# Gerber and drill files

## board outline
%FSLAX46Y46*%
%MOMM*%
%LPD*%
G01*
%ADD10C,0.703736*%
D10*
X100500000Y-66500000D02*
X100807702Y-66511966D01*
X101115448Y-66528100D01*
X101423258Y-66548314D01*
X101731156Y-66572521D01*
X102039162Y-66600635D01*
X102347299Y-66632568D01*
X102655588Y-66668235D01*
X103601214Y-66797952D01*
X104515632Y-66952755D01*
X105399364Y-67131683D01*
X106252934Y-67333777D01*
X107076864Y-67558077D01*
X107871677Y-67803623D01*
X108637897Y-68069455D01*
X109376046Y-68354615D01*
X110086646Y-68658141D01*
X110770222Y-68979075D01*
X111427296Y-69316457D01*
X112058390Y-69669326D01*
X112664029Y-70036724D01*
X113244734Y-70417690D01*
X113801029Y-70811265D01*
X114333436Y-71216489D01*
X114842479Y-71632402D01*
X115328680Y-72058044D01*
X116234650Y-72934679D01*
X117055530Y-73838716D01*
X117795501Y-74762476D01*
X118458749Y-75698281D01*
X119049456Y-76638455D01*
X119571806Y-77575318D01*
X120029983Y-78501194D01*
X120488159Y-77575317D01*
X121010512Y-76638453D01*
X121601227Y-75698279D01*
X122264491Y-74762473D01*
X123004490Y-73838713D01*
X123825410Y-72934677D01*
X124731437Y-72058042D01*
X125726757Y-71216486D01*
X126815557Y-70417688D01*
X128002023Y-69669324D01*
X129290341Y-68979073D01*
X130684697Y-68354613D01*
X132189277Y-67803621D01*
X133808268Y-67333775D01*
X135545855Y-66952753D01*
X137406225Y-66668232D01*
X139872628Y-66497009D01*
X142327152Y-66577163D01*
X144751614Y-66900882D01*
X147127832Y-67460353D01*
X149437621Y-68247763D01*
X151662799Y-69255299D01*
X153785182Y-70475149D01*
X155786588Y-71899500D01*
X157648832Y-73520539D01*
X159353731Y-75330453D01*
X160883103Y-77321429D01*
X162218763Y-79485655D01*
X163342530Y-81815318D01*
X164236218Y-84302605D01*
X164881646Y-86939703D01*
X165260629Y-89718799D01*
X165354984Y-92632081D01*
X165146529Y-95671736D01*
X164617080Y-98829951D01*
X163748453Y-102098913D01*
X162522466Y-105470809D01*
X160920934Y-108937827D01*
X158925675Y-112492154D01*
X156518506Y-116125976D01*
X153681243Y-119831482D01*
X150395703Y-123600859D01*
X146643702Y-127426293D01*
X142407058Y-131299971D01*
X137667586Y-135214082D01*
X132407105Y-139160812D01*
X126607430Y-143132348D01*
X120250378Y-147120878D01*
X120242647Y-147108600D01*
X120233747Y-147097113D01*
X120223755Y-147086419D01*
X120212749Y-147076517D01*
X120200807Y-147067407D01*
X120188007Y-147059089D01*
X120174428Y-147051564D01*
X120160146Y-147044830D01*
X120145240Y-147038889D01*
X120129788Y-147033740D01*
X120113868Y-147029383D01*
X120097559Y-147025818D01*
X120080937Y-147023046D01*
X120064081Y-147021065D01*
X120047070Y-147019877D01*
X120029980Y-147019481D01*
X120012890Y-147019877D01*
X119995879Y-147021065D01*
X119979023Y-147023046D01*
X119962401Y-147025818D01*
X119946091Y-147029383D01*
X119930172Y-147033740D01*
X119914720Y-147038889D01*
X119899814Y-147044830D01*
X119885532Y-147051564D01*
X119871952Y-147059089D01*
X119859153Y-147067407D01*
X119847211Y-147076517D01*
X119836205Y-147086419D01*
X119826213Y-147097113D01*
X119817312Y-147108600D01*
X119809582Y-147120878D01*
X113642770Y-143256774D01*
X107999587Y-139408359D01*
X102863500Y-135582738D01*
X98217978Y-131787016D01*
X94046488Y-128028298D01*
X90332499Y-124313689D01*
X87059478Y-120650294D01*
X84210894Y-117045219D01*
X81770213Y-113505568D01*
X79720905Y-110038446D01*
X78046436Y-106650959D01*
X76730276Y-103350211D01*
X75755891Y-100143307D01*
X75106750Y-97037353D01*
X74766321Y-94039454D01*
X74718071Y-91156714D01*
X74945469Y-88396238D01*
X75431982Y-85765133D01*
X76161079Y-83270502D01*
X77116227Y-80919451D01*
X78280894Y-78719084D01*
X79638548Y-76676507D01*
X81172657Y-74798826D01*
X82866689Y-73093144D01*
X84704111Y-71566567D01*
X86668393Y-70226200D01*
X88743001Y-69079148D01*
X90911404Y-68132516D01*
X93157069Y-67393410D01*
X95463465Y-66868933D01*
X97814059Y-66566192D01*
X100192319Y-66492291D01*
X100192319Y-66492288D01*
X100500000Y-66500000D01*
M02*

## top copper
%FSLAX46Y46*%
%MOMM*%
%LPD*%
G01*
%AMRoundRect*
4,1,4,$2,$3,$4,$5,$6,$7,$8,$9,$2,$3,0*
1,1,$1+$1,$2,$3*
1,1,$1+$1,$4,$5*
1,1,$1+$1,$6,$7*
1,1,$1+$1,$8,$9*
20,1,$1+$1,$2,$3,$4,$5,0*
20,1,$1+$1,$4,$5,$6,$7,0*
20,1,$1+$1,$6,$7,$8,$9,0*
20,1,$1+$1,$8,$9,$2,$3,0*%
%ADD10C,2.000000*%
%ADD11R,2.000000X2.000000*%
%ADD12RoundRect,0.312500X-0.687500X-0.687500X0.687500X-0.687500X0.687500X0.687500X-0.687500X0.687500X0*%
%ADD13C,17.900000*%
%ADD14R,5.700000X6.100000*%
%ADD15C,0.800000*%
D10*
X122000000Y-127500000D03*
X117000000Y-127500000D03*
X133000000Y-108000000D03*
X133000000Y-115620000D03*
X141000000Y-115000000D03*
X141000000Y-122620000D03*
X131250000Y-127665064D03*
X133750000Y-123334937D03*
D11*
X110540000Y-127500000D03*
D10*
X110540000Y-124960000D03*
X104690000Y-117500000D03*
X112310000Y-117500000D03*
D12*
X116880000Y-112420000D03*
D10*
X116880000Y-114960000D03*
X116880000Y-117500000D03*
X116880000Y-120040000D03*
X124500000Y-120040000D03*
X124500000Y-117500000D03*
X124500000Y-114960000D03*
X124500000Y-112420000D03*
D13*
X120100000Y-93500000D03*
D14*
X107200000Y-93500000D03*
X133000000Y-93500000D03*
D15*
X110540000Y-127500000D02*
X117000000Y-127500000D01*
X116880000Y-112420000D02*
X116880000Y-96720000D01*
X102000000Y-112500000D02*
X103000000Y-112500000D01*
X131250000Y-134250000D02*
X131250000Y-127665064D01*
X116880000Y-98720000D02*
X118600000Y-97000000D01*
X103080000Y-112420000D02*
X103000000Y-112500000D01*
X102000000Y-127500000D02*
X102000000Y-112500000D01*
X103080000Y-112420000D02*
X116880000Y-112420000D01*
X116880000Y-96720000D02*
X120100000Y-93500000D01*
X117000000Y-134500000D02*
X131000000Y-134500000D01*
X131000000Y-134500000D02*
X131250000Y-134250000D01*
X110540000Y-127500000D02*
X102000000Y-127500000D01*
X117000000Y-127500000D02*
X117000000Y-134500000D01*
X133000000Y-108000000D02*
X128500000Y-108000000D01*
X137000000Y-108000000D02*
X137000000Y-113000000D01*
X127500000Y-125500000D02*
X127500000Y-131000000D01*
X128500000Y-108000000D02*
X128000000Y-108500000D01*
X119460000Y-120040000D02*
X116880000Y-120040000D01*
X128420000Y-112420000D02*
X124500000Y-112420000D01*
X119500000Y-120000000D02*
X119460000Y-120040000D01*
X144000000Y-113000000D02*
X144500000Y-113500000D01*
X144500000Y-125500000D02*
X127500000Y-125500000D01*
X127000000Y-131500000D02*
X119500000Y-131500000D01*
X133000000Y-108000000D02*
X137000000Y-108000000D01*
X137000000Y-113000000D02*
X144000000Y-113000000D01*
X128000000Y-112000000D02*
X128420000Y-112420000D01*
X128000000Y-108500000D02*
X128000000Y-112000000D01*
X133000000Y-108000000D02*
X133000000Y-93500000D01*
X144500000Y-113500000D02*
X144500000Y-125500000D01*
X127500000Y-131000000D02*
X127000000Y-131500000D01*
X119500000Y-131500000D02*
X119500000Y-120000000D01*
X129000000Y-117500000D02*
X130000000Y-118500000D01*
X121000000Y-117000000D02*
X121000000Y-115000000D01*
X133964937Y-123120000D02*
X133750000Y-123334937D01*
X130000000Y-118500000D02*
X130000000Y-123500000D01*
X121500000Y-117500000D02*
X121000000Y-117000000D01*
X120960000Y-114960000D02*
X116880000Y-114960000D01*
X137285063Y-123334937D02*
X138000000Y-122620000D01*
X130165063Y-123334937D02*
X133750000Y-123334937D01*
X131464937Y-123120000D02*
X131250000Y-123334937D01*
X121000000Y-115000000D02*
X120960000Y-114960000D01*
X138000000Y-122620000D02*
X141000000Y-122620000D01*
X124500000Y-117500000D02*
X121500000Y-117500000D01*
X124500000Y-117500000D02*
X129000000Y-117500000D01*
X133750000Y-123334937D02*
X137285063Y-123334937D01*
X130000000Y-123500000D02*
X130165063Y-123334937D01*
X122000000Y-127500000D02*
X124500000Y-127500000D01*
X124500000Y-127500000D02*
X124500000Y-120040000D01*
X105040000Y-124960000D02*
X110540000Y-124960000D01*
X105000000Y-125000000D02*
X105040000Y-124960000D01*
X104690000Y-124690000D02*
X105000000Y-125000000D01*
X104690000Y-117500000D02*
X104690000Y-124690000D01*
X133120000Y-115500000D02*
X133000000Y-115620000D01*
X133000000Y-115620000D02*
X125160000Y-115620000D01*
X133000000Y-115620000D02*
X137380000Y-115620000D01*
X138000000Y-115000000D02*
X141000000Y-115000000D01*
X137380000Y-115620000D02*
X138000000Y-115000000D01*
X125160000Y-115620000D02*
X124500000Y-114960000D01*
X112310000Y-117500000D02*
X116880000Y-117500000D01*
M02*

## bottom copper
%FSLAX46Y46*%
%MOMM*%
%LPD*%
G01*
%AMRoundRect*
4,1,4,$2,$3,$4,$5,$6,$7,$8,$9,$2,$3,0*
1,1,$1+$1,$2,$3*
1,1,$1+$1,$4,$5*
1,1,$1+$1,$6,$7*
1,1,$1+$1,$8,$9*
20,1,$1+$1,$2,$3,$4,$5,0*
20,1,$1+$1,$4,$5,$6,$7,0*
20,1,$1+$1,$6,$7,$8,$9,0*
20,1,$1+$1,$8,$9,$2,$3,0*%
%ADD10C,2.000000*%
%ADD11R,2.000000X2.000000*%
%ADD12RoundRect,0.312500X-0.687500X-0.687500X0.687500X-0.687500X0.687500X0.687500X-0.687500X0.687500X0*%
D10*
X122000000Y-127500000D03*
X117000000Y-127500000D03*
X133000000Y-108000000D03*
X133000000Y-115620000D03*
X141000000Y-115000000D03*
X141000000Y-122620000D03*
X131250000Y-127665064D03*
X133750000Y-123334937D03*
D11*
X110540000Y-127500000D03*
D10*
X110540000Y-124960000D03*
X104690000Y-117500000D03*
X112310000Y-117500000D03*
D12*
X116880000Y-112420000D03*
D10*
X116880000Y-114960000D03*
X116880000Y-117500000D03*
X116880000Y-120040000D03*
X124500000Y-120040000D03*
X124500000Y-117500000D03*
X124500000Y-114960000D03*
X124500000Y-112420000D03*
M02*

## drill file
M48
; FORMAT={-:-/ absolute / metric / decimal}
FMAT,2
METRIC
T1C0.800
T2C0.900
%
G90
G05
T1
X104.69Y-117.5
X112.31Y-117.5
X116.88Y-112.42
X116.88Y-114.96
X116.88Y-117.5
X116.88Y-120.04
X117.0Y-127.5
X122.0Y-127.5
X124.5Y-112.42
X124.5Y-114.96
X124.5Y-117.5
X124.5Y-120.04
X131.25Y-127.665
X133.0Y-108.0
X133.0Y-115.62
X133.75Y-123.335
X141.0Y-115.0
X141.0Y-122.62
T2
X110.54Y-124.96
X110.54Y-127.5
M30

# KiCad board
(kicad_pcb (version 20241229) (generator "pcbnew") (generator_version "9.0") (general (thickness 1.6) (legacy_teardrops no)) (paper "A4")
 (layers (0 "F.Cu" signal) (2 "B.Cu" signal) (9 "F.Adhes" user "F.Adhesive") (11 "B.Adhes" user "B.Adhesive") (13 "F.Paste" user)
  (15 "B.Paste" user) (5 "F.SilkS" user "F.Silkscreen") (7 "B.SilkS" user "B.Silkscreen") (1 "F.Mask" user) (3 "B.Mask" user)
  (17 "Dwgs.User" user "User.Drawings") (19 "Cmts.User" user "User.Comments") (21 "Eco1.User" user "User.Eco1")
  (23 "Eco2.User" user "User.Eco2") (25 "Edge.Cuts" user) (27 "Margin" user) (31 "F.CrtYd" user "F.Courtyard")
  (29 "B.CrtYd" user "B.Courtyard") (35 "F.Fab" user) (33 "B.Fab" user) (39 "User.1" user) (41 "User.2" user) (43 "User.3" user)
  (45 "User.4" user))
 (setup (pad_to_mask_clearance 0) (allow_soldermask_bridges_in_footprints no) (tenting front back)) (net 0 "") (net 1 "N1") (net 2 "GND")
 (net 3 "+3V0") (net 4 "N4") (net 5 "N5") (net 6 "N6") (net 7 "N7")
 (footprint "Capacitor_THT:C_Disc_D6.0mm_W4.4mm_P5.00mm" (layer "F.Cu") (at 122 127.5 180)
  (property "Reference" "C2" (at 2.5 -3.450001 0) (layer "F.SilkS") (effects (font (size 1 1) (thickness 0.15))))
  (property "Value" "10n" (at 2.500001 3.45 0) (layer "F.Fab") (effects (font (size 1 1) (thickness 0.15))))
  (pad "1" thru_hole circle (at 0 0 180) (size 2 2) (drill 0.8) (layers "*.Cu" "*.Mask") (remove_unused_layers no) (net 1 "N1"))
  (pad "2" thru_hole circle (at 5 0 180) (size 2 2) (drill 0.8) (layers "*.Cu" "*.Mask") (remove_unused_layers no) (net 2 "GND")))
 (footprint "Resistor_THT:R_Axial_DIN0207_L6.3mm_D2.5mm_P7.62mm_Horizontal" (layer "F.Cu") (at 133 108 -90)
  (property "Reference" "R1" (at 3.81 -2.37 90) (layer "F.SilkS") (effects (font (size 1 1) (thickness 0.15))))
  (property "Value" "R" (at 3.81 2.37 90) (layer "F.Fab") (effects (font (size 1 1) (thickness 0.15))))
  (pad "1" thru_hole circle (at 0 0 270) (size 2 2) (drill 0.8) (layers "*.Cu" "*.Mask") (remove_unused_layers no) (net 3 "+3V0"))
  (pad "2" thru_hole circle (at 7.62 0 270) (size 2 2) (drill 0.8) (layers "*.Cu" "*.Mask") (remove_unused_layers no) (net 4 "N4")))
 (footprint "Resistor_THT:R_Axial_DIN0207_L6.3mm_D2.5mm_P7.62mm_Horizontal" (layer "F.Cu") (at 141 115 -90)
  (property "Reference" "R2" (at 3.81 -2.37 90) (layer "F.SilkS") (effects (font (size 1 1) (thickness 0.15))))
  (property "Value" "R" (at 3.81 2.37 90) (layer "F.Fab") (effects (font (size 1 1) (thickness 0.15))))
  (pad "1" thru_hole circle (at 0 0 270) (size 2 2) (drill 0.8) (layers "*.Cu" "*.Mask") (remove_unused_layers no) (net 4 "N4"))
  (pad "2" thru_hole circle (at 7.62 0 270) (size 2 2) (drill 0.8) (layers "*.Cu" "*.Mask") (remove_unused_layers no) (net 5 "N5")))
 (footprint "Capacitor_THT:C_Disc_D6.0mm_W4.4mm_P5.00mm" (layer "F.Cu") (at 131.25 127.665064 60)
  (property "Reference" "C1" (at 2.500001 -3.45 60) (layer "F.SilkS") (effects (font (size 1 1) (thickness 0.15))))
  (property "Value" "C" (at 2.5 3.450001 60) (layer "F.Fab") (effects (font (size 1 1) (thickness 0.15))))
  (pad "1" thru_hole circle (at 0 0 60) (size 2 2) (drill 0.8) (layers "*.Cu" "*.Mask") (remove_unused_layers no) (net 2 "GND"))
  (pad "2" thru_hole circle (at 5 0 60) (size 2 2) (drill 0.8) (layers "*.Cu" "*.Mask") (remove_unused_layers no) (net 5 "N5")))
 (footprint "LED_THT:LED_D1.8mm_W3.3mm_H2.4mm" (layer "F.Cu") (at 110.54 127.5 90)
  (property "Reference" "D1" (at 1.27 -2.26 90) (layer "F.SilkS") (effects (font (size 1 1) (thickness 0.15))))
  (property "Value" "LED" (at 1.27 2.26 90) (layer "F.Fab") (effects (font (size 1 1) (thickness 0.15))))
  (pad "1" thru_hole rect (at 0 0 90) (size 2 2) (drill 0.9) (layers "*.Cu" "*.Mask") (remove_unused_layers no) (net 2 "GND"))
  (pad "2" thru_hole circle (at 2.54 0 90) (size 2 2) (drill 0.9) (layers "*.Cu" "*.Mask") (remove_unused_layers no) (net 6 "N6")))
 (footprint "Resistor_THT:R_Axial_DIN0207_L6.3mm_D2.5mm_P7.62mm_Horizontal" (layer "F.Cu") (at 104.69 117.5)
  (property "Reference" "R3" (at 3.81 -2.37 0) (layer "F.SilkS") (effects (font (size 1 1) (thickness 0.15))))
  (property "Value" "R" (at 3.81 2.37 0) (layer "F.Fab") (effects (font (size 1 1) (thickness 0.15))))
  (pad "1" thru_hole circle (at 0 0) (size 2 2) (drill 0.8) (layers "*.Cu" "*.Mask") (remove_unused_layers no) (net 6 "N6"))
  (pad "2" thru_hole circle (at 7.62 0) (size 2 2) (drill 0.8) (layers "*.Cu" "*.Mask") (remove_unused_layers no) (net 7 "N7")))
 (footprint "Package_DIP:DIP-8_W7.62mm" (layer "F.Cu") (at 116.88 112.42)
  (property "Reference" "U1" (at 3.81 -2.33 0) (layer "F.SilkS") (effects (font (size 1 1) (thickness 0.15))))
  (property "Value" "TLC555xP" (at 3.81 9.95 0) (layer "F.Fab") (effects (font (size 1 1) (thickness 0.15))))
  (pad "1" thru_hole roundrect (at 0 0) (size 2 2) (drill 0.8) (layers "*.Cu" "*.Mask") (remove_unused_layers no) (roundrect_rratio 0.15625)
   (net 2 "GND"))
  (pad "2" thru_hole circle (at 0 2.54) (size 2 2) (drill 0.8) (layers "*.Cu" "*.Mask") (remove_unused_layers no) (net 5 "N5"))
  (pad "3" thru_hole circle (at 0 5.08) (size 2 2) (drill 0.8) (layers "*.Cu" "*.Mask") (remove_unused_layers no) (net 7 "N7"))
  (pad "4" thru_hole circle (at 0 7.62) (size 2 2) (drill 0.8) (layers "*.Cu" "*.Mask") (remove_unused_layers no) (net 3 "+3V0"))
  (pad "5" thru_hole circle (at 7.62 7.62) (size 2 2) (drill 0.8) (layers "*.Cu" "*.Mask") (remove_unused_layers no) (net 1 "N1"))
  (pad "6" thru_hole circle (at 7.62 5.08) (size 2 2) (drill 0.8) (layers "*.Cu" "*.Mask") (remove_unused_layers no) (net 5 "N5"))
  (pad "7" thru_hole circle (at 7.62 2.54) (size 2 2) (drill 0.8) (layers "*.Cu" "*.Mask") (remove_unused_layers no) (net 4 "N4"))
  (pad "8" thru_hole circle (at 7.62 0) (size 2 2) (drill 0.8) (layers "*.Cu" "*.Mask") (remove_unused_layers no) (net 3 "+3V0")))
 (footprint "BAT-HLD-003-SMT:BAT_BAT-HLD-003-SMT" (layer "F.Cu") (at 120.1 93.5)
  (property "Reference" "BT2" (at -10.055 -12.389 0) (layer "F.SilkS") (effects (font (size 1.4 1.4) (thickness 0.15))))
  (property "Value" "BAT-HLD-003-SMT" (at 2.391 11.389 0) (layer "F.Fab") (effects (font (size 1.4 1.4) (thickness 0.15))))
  (pad "N" smd circle (at 0 0) (size 17.9 17.9) (layers "F.Cu" "F.Mask") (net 2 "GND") (solder_mask_margin 0.102))
  (pad "P1" smd rect (at -12.9 0) (size 5.7 6.1) (layers "F.Cu" "F.Mask" "F.Paste") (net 3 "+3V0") (solder_mask_margin 0.102))
  (pad "P2" smd rect (at 12.9 0) (size 5.7 6.1) (layers "F.Cu" "F.Mask" "F.Paste") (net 3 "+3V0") (solder_mask_margin 0.102)))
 (gr_poly
  (pts (xy 100.5 66.5) (xy 100.807702 66.511966) (xy 101.115448 66.5281) (xy 101.423258 66.548314) (xy 101.731156 66.572521)
   (xy 102.039162 66.600635) (xy 102.347299 66.632568) (xy 102.655588 66.668235) (xy 103.601214 66.797952) (xy 104.515632 66.952755)
   (xy 105.399364 67.131683) (xy 106.252934 67.333777) (xy 107.076864 67.558077) (xy 107.871677 67.803623) (xy 108.637897 68.069455)
   (xy 109.376046 68.354615) (xy 110.086646 68.658141) (xy 110.770222 68.979075) (xy 111.427296 69.316457) (xy 112.05839 69.669326)
   (xy 112.664029 70.036724) (xy 113.244734 70.41769) (xy 113.801029 70.811265) (xy 114.333436 71.216489) (xy 114.842479 71.632402)
   (xy 115.32868 72.058044) (xy 116.23465 72.934679) (xy 117.05553 73.838716) (xy 117.795501 74.762476) (xy 118.458749 75.698281)
   (xy 119.049456 76.638455) (xy 119.571806 77.575318) (xy 120.029983 78.501194) (xy 120.488159 77.575317) (xy 121.010512 76.638453)
   (xy 121.601227 75.698279) (xy 122.264491 74.762473) (xy 123.00449 73.838713) (xy 123.82541 72.934677) (xy 124.731437 72.058042)
   (xy 125.726757 71.216486) (xy 126.815557 70.417688) (xy 128.002023 69.669324) (xy 129.290341 68.979073) (xy 130.684697 68.354613)
   (xy 132.189277 67.803621) (xy 133.808268 67.333775) (xy 135.545855 66.952753) (xy 137.406225 66.668232) (xy 139.872628 66.497009)
   (xy 142.327152 66.577163) (xy 144.751614 66.900882) (xy 147.127832 67.460353) (xy 149.437621 68.247763) (xy 151.662799 69.255299)
   (xy 153.785182 70.475149) (xy 155.786588 71.8995) (xy 157.648832 73.520539) (xy 159.353731 75.330453) (xy 160.883103 77.321429)
   (xy 162.218763 79.485655) (xy 163.34253 81.815318) (xy 164.236218 84.302605) (xy 164.881646 86.939703) (xy 165.260629 89.718799)
   (xy 165.354984 92.632081) (xy 165.146529 95.671736) (xy 164.61708 98.829951) (xy 163.748453 102.098913) (xy 162.522466 105.470809)
   (xy 160.920934 108.937827) (xy 158.925675 112.492154) (xy 156.518506 116.125976) (xy 153.681243 119.831482) (xy 150.395703 123.600859)
   (xy 146.643702 127.426293) (xy 142.407058 131.299971) (xy 137.667586 135.214082) (xy 132.407105 139.160812) (xy 126.60743 143.132348)
   (xy 120.250378 147.120878) (xy 120.242647 147.1086) (xy 120.233747 147.097113) (xy 120.223755 147.086419) (xy 120.212749 147.076517)
   (xy 120.200807 147.067407) (xy 120.188007 147.059089) (xy 120.174428 147.051564) (xy 120.160146 147.04483) (xy 120.14524 147.038889)
   (xy 120.129788 147.03374) (xy 120.113868 147.029383) (xy 120.097559 147.025818) (xy 120.080937 147.023046) (xy 120.064081 147.021065)
   (xy 120.04707 147.019877) (xy 120.02998 147.019481) (xy 120.01289 147.019877) (xy 119.995879 147.021065) (xy 119.979023 147.023046)
   (xy 119.962401 147.025818) (xy 119.946091 147.029383) (xy 119.930172 147.03374) (xy 119.91472 147.038889) (xy 119.899814 147.04483)
   (xy 119.885532 147.051564) (xy 119.871952 147.059089) (xy 119.859153 147.067407) (xy 119.847211 147.076517) (xy 119.836205 147.086419)
   (xy 119.826213 147.097113) (xy 119.817312 147.1086) (xy 119.809582 147.120878) (xy 113.64277 143.256774) (xy 107.999587 139.408359)
   (xy 102.8635 135.582738) (xy 98.217978 131.787016) (xy 94.046488 128.028298) (xy 90.332499 124.313689) (xy 87.059478 120.650294)
   (xy 84.210894 117.045219) (xy 81.770213 113.505568) (xy 79.720905 110.038446) (xy 78.046436 106.650959) (xy 76.730276 103.350211)
   (xy 75.755891 100.143307) (xy 75.10675 97.037353) (xy 74.766321 94.039454) (xy 74.718071 91.156714) (xy 74.945469 88.396238)
   (xy 75.431982 85.765133) (xy 76.161079 83.270502) (xy 77.116227 80.919451) (xy 78.280894 78.719084) (xy 79.638548 76.676507)
   (xy 81.172657 74.798826) (xy 82.866689 73.093144) (xy 84.704111 71.566567) (xy 86.668393 70.2262) (xy 88.743001 69.079148)
   (xy 90.911404 68.132516) (xy 93.157069 67.39341) (xy 95.463465 66.868933) (xy 97.814059 66.566192) (xy 100.192319 66.492291)
   (xy 100.192319 66.492288))
  (stroke (width 0.703736) (type solid)) (fill no) (layer "Edge.Cuts"))
 (segment (start 110.54 127.5) (end 117 127.5) (width 0.8) (layer "F.Cu") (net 2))
 (segment (start 116.88 112.42) (end 116.88 96.72) (width 0.8) (layer "F.Cu") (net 2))
 (segment (start 102 112.5) (end 103 112.5) (width 0.8) (layer "F.Cu") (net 2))
 (segment (start 131.25 134.25) (end 131.25 127.665064) (width 0.8) (layer "F.Cu") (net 2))
 (segment (start 116.88 98.72) (end 118.6 97) (width 0.8) (layer "F.Cu") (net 2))
 (segment (start 103.08 112.42) (end 103 112.5) (width 0.8) (layer "F.Cu") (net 2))
 (segment (start 102 127.5) (end 102 112.5) (width 0.8) (layer "F.Cu") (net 2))
 (segment (start 103.08 112.42) (end 116.88 112.42) (width 0.8) (layer "F.Cu") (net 2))
 (segment (start 116.88 96.72) (end 120.1 93.5) (width 0.8) (layer "F.Cu") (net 2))
 (segment (start 117 134.5) (end 131 134.5) (width 0.8) (layer "F.Cu") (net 2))
 (segment (start 131 134.5) (end 131.25 134.25) (width 0.8) (layer "F.Cu") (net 2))
 (segment (start 110.54 127.5) (end 102 127.5) (width 0.8) (layer "F.Cu") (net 2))
 (segment (start 117 127.5) (end 117 134.5) (width 0.8) (layer "F.Cu") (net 2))
 (segment (start 133 108) (end 128.5 108) (width 0.8) (layer "F.Cu") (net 3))
 (segment (start 137 108) (end 137 113) (width 0.8) (layer "F.Cu") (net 3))
 (segment (start 127.5 125.5) (end 127.5 131) (width 0.8) (layer "F.Cu") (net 3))
 (segment (start 128.5 108) (end 128 108.5) (width 0.8) (layer "F.Cu") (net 3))
 (segment (start 119.46 120.04) (end 116.88 120.04) (width 0.8) (layer "F.Cu") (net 3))
 (segment (start 128.42 112.42) (end 124.5 112.42) (width 0.8) (layer "F.Cu") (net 3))
 (segment (start 119.5 120) (end 119.46 120.04) (width 0.8) (layer "F.Cu") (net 3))
 (segment (start 144 113) (end 144.5 113.5) (width 0.8) (layer "F.Cu") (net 3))
 (segment (start 144.5 125.5) (end 127.5 125.5) (width 0.8) (layer "F.Cu") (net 3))
 (segment (start 127 131.5) (end 119.5 131.5) (width 0.8) (layer "F.Cu") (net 3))
 (segment (start 133 108) (end 137 108) (width 0.8) (layer "F.Cu") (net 3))
 (segment (start 137 113) (end 144 113) (width 0.8) (layer "F.Cu") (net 3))
 (segment (start 128 112) (end 128.42 112.42) (width 0.8) (layer "F.Cu") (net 3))
 (segment (start 128 108.5) (end 128 112) (width 0.8) (layer "F.Cu") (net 3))
 (segment (start 133 108) (end 133 93.5) (width 0.8) (layer "F.Cu") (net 3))
 (segment (start 144.5 113.5) (end 144.5 125.5) (width 0.8) (layer "F.Cu") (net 3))
 (segment (start 127.5 131) (end 127 131.5) (width 0.8) (layer "F.Cu") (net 3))
 (segment (start 119.5 131.5) (end 119.5 120) (width 0.8) (layer "F.Cu") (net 3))
 (segment (start 129 117.5) (end 130 118.5) (width 0.8) (layer "F.Cu") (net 5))
 (segment (start 121 117) (end 121 115) (width 0.8) (layer "F.Cu") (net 5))
 (segment (start 133.964937 123.12) (end 133.75 123.334937) (width 0.8) (layer "F.Cu") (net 5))
 (segment (start 130 118.5) (end 130 123.5) (width 0.8) (layer "F.Cu") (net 5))
 (segment (start 121.5 117.5) (end 121 117) (width 0.8) (layer "F.Cu") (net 5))
 (segment (start 120.96 114.96) (end 116.88 114.96) (width 0.8) (layer "F.Cu") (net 5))
 (segment (start 137.285063 123.334937) (end 138 122.62) (width 0.8) (layer "F.Cu") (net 5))
 (segment (start 130.165063 123.334937) (end 133.75 123.334937) (width 0.8) (layer "F.Cu") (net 5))
 (segment (start 131.464937 123.12) (end 131.25 123.334937) (width 0.8) (layer "F.Cu") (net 5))
 (segment (start 121 115) (end 120.96 114.96) (width 0.8) (layer "F.Cu") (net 5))
 (segment (start 138 122.62) (end 141 122.62) (width 0.8) (layer "F.Cu") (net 5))
 (segment (start 124.5 117.5) (end 121.5 117.5) (width 0.8) (layer "F.Cu") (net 5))
 (segment (start 124.5 117.5) (end 129 117.5) (width 0.8) (layer "F.Cu") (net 5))
 (segment (start 133.75 123.334937) (end 137.285063 123.334937) (width 0.8) (layer "F.Cu") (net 5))
 (segment (start 130 123.5) (end 130.165063 123.334937) (width 0.8) (layer "F.Cu") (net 5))
 (segment (start 122 127.5) (end 124.5 127.5) (width 0.8) (layer "F.Cu") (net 1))
 (segment (start 124.5 127.5) (end 124.5 120.04) (width 0.8) (layer "F.Cu") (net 1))
 (segment (start 105.04 124.96) (end 110.54 124.96) (width 0.8) (layer "F.Cu") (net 6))
 (segment (start 105 125) (end 105.04 124.96) (width 0.8) (layer "F.Cu") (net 6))
 (segment (start 104.69 124.69) (end 105 125) (width 0.8) (layer "F.Cu") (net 6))
 (segment (start 104.69 117.5) (end 104.69 124.69) (width 0.8) (layer "F.Cu") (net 6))
 (segment (start 133.12 115.5) (end 133 115.62) (width 0.8) (layer "F.Cu") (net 4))
 (segment (start 133 115.62) (end 125.16 115.62) (width 0.8) (layer "F.Cu") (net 4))
 (segment (start 133 115.62) (end 137.38 115.62) (width 0.8) (layer "F.Cu") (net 4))
 (segment (start 138 115) (end 141 115) (width 0.8) (layer "F.Cu") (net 4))
 (segment (start 137.38 115.62) (end 138 115) (width 0.8) (layer "F.Cu") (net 4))
 (segment (start 125.16 115.62) (end 124.5 114.96) (width 0.8) (layer "F.Cu") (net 4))
 (segment (start 112.31 117.5) (end 116.88 117.5) (width 0.8) (layer "F.Cu") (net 7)))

